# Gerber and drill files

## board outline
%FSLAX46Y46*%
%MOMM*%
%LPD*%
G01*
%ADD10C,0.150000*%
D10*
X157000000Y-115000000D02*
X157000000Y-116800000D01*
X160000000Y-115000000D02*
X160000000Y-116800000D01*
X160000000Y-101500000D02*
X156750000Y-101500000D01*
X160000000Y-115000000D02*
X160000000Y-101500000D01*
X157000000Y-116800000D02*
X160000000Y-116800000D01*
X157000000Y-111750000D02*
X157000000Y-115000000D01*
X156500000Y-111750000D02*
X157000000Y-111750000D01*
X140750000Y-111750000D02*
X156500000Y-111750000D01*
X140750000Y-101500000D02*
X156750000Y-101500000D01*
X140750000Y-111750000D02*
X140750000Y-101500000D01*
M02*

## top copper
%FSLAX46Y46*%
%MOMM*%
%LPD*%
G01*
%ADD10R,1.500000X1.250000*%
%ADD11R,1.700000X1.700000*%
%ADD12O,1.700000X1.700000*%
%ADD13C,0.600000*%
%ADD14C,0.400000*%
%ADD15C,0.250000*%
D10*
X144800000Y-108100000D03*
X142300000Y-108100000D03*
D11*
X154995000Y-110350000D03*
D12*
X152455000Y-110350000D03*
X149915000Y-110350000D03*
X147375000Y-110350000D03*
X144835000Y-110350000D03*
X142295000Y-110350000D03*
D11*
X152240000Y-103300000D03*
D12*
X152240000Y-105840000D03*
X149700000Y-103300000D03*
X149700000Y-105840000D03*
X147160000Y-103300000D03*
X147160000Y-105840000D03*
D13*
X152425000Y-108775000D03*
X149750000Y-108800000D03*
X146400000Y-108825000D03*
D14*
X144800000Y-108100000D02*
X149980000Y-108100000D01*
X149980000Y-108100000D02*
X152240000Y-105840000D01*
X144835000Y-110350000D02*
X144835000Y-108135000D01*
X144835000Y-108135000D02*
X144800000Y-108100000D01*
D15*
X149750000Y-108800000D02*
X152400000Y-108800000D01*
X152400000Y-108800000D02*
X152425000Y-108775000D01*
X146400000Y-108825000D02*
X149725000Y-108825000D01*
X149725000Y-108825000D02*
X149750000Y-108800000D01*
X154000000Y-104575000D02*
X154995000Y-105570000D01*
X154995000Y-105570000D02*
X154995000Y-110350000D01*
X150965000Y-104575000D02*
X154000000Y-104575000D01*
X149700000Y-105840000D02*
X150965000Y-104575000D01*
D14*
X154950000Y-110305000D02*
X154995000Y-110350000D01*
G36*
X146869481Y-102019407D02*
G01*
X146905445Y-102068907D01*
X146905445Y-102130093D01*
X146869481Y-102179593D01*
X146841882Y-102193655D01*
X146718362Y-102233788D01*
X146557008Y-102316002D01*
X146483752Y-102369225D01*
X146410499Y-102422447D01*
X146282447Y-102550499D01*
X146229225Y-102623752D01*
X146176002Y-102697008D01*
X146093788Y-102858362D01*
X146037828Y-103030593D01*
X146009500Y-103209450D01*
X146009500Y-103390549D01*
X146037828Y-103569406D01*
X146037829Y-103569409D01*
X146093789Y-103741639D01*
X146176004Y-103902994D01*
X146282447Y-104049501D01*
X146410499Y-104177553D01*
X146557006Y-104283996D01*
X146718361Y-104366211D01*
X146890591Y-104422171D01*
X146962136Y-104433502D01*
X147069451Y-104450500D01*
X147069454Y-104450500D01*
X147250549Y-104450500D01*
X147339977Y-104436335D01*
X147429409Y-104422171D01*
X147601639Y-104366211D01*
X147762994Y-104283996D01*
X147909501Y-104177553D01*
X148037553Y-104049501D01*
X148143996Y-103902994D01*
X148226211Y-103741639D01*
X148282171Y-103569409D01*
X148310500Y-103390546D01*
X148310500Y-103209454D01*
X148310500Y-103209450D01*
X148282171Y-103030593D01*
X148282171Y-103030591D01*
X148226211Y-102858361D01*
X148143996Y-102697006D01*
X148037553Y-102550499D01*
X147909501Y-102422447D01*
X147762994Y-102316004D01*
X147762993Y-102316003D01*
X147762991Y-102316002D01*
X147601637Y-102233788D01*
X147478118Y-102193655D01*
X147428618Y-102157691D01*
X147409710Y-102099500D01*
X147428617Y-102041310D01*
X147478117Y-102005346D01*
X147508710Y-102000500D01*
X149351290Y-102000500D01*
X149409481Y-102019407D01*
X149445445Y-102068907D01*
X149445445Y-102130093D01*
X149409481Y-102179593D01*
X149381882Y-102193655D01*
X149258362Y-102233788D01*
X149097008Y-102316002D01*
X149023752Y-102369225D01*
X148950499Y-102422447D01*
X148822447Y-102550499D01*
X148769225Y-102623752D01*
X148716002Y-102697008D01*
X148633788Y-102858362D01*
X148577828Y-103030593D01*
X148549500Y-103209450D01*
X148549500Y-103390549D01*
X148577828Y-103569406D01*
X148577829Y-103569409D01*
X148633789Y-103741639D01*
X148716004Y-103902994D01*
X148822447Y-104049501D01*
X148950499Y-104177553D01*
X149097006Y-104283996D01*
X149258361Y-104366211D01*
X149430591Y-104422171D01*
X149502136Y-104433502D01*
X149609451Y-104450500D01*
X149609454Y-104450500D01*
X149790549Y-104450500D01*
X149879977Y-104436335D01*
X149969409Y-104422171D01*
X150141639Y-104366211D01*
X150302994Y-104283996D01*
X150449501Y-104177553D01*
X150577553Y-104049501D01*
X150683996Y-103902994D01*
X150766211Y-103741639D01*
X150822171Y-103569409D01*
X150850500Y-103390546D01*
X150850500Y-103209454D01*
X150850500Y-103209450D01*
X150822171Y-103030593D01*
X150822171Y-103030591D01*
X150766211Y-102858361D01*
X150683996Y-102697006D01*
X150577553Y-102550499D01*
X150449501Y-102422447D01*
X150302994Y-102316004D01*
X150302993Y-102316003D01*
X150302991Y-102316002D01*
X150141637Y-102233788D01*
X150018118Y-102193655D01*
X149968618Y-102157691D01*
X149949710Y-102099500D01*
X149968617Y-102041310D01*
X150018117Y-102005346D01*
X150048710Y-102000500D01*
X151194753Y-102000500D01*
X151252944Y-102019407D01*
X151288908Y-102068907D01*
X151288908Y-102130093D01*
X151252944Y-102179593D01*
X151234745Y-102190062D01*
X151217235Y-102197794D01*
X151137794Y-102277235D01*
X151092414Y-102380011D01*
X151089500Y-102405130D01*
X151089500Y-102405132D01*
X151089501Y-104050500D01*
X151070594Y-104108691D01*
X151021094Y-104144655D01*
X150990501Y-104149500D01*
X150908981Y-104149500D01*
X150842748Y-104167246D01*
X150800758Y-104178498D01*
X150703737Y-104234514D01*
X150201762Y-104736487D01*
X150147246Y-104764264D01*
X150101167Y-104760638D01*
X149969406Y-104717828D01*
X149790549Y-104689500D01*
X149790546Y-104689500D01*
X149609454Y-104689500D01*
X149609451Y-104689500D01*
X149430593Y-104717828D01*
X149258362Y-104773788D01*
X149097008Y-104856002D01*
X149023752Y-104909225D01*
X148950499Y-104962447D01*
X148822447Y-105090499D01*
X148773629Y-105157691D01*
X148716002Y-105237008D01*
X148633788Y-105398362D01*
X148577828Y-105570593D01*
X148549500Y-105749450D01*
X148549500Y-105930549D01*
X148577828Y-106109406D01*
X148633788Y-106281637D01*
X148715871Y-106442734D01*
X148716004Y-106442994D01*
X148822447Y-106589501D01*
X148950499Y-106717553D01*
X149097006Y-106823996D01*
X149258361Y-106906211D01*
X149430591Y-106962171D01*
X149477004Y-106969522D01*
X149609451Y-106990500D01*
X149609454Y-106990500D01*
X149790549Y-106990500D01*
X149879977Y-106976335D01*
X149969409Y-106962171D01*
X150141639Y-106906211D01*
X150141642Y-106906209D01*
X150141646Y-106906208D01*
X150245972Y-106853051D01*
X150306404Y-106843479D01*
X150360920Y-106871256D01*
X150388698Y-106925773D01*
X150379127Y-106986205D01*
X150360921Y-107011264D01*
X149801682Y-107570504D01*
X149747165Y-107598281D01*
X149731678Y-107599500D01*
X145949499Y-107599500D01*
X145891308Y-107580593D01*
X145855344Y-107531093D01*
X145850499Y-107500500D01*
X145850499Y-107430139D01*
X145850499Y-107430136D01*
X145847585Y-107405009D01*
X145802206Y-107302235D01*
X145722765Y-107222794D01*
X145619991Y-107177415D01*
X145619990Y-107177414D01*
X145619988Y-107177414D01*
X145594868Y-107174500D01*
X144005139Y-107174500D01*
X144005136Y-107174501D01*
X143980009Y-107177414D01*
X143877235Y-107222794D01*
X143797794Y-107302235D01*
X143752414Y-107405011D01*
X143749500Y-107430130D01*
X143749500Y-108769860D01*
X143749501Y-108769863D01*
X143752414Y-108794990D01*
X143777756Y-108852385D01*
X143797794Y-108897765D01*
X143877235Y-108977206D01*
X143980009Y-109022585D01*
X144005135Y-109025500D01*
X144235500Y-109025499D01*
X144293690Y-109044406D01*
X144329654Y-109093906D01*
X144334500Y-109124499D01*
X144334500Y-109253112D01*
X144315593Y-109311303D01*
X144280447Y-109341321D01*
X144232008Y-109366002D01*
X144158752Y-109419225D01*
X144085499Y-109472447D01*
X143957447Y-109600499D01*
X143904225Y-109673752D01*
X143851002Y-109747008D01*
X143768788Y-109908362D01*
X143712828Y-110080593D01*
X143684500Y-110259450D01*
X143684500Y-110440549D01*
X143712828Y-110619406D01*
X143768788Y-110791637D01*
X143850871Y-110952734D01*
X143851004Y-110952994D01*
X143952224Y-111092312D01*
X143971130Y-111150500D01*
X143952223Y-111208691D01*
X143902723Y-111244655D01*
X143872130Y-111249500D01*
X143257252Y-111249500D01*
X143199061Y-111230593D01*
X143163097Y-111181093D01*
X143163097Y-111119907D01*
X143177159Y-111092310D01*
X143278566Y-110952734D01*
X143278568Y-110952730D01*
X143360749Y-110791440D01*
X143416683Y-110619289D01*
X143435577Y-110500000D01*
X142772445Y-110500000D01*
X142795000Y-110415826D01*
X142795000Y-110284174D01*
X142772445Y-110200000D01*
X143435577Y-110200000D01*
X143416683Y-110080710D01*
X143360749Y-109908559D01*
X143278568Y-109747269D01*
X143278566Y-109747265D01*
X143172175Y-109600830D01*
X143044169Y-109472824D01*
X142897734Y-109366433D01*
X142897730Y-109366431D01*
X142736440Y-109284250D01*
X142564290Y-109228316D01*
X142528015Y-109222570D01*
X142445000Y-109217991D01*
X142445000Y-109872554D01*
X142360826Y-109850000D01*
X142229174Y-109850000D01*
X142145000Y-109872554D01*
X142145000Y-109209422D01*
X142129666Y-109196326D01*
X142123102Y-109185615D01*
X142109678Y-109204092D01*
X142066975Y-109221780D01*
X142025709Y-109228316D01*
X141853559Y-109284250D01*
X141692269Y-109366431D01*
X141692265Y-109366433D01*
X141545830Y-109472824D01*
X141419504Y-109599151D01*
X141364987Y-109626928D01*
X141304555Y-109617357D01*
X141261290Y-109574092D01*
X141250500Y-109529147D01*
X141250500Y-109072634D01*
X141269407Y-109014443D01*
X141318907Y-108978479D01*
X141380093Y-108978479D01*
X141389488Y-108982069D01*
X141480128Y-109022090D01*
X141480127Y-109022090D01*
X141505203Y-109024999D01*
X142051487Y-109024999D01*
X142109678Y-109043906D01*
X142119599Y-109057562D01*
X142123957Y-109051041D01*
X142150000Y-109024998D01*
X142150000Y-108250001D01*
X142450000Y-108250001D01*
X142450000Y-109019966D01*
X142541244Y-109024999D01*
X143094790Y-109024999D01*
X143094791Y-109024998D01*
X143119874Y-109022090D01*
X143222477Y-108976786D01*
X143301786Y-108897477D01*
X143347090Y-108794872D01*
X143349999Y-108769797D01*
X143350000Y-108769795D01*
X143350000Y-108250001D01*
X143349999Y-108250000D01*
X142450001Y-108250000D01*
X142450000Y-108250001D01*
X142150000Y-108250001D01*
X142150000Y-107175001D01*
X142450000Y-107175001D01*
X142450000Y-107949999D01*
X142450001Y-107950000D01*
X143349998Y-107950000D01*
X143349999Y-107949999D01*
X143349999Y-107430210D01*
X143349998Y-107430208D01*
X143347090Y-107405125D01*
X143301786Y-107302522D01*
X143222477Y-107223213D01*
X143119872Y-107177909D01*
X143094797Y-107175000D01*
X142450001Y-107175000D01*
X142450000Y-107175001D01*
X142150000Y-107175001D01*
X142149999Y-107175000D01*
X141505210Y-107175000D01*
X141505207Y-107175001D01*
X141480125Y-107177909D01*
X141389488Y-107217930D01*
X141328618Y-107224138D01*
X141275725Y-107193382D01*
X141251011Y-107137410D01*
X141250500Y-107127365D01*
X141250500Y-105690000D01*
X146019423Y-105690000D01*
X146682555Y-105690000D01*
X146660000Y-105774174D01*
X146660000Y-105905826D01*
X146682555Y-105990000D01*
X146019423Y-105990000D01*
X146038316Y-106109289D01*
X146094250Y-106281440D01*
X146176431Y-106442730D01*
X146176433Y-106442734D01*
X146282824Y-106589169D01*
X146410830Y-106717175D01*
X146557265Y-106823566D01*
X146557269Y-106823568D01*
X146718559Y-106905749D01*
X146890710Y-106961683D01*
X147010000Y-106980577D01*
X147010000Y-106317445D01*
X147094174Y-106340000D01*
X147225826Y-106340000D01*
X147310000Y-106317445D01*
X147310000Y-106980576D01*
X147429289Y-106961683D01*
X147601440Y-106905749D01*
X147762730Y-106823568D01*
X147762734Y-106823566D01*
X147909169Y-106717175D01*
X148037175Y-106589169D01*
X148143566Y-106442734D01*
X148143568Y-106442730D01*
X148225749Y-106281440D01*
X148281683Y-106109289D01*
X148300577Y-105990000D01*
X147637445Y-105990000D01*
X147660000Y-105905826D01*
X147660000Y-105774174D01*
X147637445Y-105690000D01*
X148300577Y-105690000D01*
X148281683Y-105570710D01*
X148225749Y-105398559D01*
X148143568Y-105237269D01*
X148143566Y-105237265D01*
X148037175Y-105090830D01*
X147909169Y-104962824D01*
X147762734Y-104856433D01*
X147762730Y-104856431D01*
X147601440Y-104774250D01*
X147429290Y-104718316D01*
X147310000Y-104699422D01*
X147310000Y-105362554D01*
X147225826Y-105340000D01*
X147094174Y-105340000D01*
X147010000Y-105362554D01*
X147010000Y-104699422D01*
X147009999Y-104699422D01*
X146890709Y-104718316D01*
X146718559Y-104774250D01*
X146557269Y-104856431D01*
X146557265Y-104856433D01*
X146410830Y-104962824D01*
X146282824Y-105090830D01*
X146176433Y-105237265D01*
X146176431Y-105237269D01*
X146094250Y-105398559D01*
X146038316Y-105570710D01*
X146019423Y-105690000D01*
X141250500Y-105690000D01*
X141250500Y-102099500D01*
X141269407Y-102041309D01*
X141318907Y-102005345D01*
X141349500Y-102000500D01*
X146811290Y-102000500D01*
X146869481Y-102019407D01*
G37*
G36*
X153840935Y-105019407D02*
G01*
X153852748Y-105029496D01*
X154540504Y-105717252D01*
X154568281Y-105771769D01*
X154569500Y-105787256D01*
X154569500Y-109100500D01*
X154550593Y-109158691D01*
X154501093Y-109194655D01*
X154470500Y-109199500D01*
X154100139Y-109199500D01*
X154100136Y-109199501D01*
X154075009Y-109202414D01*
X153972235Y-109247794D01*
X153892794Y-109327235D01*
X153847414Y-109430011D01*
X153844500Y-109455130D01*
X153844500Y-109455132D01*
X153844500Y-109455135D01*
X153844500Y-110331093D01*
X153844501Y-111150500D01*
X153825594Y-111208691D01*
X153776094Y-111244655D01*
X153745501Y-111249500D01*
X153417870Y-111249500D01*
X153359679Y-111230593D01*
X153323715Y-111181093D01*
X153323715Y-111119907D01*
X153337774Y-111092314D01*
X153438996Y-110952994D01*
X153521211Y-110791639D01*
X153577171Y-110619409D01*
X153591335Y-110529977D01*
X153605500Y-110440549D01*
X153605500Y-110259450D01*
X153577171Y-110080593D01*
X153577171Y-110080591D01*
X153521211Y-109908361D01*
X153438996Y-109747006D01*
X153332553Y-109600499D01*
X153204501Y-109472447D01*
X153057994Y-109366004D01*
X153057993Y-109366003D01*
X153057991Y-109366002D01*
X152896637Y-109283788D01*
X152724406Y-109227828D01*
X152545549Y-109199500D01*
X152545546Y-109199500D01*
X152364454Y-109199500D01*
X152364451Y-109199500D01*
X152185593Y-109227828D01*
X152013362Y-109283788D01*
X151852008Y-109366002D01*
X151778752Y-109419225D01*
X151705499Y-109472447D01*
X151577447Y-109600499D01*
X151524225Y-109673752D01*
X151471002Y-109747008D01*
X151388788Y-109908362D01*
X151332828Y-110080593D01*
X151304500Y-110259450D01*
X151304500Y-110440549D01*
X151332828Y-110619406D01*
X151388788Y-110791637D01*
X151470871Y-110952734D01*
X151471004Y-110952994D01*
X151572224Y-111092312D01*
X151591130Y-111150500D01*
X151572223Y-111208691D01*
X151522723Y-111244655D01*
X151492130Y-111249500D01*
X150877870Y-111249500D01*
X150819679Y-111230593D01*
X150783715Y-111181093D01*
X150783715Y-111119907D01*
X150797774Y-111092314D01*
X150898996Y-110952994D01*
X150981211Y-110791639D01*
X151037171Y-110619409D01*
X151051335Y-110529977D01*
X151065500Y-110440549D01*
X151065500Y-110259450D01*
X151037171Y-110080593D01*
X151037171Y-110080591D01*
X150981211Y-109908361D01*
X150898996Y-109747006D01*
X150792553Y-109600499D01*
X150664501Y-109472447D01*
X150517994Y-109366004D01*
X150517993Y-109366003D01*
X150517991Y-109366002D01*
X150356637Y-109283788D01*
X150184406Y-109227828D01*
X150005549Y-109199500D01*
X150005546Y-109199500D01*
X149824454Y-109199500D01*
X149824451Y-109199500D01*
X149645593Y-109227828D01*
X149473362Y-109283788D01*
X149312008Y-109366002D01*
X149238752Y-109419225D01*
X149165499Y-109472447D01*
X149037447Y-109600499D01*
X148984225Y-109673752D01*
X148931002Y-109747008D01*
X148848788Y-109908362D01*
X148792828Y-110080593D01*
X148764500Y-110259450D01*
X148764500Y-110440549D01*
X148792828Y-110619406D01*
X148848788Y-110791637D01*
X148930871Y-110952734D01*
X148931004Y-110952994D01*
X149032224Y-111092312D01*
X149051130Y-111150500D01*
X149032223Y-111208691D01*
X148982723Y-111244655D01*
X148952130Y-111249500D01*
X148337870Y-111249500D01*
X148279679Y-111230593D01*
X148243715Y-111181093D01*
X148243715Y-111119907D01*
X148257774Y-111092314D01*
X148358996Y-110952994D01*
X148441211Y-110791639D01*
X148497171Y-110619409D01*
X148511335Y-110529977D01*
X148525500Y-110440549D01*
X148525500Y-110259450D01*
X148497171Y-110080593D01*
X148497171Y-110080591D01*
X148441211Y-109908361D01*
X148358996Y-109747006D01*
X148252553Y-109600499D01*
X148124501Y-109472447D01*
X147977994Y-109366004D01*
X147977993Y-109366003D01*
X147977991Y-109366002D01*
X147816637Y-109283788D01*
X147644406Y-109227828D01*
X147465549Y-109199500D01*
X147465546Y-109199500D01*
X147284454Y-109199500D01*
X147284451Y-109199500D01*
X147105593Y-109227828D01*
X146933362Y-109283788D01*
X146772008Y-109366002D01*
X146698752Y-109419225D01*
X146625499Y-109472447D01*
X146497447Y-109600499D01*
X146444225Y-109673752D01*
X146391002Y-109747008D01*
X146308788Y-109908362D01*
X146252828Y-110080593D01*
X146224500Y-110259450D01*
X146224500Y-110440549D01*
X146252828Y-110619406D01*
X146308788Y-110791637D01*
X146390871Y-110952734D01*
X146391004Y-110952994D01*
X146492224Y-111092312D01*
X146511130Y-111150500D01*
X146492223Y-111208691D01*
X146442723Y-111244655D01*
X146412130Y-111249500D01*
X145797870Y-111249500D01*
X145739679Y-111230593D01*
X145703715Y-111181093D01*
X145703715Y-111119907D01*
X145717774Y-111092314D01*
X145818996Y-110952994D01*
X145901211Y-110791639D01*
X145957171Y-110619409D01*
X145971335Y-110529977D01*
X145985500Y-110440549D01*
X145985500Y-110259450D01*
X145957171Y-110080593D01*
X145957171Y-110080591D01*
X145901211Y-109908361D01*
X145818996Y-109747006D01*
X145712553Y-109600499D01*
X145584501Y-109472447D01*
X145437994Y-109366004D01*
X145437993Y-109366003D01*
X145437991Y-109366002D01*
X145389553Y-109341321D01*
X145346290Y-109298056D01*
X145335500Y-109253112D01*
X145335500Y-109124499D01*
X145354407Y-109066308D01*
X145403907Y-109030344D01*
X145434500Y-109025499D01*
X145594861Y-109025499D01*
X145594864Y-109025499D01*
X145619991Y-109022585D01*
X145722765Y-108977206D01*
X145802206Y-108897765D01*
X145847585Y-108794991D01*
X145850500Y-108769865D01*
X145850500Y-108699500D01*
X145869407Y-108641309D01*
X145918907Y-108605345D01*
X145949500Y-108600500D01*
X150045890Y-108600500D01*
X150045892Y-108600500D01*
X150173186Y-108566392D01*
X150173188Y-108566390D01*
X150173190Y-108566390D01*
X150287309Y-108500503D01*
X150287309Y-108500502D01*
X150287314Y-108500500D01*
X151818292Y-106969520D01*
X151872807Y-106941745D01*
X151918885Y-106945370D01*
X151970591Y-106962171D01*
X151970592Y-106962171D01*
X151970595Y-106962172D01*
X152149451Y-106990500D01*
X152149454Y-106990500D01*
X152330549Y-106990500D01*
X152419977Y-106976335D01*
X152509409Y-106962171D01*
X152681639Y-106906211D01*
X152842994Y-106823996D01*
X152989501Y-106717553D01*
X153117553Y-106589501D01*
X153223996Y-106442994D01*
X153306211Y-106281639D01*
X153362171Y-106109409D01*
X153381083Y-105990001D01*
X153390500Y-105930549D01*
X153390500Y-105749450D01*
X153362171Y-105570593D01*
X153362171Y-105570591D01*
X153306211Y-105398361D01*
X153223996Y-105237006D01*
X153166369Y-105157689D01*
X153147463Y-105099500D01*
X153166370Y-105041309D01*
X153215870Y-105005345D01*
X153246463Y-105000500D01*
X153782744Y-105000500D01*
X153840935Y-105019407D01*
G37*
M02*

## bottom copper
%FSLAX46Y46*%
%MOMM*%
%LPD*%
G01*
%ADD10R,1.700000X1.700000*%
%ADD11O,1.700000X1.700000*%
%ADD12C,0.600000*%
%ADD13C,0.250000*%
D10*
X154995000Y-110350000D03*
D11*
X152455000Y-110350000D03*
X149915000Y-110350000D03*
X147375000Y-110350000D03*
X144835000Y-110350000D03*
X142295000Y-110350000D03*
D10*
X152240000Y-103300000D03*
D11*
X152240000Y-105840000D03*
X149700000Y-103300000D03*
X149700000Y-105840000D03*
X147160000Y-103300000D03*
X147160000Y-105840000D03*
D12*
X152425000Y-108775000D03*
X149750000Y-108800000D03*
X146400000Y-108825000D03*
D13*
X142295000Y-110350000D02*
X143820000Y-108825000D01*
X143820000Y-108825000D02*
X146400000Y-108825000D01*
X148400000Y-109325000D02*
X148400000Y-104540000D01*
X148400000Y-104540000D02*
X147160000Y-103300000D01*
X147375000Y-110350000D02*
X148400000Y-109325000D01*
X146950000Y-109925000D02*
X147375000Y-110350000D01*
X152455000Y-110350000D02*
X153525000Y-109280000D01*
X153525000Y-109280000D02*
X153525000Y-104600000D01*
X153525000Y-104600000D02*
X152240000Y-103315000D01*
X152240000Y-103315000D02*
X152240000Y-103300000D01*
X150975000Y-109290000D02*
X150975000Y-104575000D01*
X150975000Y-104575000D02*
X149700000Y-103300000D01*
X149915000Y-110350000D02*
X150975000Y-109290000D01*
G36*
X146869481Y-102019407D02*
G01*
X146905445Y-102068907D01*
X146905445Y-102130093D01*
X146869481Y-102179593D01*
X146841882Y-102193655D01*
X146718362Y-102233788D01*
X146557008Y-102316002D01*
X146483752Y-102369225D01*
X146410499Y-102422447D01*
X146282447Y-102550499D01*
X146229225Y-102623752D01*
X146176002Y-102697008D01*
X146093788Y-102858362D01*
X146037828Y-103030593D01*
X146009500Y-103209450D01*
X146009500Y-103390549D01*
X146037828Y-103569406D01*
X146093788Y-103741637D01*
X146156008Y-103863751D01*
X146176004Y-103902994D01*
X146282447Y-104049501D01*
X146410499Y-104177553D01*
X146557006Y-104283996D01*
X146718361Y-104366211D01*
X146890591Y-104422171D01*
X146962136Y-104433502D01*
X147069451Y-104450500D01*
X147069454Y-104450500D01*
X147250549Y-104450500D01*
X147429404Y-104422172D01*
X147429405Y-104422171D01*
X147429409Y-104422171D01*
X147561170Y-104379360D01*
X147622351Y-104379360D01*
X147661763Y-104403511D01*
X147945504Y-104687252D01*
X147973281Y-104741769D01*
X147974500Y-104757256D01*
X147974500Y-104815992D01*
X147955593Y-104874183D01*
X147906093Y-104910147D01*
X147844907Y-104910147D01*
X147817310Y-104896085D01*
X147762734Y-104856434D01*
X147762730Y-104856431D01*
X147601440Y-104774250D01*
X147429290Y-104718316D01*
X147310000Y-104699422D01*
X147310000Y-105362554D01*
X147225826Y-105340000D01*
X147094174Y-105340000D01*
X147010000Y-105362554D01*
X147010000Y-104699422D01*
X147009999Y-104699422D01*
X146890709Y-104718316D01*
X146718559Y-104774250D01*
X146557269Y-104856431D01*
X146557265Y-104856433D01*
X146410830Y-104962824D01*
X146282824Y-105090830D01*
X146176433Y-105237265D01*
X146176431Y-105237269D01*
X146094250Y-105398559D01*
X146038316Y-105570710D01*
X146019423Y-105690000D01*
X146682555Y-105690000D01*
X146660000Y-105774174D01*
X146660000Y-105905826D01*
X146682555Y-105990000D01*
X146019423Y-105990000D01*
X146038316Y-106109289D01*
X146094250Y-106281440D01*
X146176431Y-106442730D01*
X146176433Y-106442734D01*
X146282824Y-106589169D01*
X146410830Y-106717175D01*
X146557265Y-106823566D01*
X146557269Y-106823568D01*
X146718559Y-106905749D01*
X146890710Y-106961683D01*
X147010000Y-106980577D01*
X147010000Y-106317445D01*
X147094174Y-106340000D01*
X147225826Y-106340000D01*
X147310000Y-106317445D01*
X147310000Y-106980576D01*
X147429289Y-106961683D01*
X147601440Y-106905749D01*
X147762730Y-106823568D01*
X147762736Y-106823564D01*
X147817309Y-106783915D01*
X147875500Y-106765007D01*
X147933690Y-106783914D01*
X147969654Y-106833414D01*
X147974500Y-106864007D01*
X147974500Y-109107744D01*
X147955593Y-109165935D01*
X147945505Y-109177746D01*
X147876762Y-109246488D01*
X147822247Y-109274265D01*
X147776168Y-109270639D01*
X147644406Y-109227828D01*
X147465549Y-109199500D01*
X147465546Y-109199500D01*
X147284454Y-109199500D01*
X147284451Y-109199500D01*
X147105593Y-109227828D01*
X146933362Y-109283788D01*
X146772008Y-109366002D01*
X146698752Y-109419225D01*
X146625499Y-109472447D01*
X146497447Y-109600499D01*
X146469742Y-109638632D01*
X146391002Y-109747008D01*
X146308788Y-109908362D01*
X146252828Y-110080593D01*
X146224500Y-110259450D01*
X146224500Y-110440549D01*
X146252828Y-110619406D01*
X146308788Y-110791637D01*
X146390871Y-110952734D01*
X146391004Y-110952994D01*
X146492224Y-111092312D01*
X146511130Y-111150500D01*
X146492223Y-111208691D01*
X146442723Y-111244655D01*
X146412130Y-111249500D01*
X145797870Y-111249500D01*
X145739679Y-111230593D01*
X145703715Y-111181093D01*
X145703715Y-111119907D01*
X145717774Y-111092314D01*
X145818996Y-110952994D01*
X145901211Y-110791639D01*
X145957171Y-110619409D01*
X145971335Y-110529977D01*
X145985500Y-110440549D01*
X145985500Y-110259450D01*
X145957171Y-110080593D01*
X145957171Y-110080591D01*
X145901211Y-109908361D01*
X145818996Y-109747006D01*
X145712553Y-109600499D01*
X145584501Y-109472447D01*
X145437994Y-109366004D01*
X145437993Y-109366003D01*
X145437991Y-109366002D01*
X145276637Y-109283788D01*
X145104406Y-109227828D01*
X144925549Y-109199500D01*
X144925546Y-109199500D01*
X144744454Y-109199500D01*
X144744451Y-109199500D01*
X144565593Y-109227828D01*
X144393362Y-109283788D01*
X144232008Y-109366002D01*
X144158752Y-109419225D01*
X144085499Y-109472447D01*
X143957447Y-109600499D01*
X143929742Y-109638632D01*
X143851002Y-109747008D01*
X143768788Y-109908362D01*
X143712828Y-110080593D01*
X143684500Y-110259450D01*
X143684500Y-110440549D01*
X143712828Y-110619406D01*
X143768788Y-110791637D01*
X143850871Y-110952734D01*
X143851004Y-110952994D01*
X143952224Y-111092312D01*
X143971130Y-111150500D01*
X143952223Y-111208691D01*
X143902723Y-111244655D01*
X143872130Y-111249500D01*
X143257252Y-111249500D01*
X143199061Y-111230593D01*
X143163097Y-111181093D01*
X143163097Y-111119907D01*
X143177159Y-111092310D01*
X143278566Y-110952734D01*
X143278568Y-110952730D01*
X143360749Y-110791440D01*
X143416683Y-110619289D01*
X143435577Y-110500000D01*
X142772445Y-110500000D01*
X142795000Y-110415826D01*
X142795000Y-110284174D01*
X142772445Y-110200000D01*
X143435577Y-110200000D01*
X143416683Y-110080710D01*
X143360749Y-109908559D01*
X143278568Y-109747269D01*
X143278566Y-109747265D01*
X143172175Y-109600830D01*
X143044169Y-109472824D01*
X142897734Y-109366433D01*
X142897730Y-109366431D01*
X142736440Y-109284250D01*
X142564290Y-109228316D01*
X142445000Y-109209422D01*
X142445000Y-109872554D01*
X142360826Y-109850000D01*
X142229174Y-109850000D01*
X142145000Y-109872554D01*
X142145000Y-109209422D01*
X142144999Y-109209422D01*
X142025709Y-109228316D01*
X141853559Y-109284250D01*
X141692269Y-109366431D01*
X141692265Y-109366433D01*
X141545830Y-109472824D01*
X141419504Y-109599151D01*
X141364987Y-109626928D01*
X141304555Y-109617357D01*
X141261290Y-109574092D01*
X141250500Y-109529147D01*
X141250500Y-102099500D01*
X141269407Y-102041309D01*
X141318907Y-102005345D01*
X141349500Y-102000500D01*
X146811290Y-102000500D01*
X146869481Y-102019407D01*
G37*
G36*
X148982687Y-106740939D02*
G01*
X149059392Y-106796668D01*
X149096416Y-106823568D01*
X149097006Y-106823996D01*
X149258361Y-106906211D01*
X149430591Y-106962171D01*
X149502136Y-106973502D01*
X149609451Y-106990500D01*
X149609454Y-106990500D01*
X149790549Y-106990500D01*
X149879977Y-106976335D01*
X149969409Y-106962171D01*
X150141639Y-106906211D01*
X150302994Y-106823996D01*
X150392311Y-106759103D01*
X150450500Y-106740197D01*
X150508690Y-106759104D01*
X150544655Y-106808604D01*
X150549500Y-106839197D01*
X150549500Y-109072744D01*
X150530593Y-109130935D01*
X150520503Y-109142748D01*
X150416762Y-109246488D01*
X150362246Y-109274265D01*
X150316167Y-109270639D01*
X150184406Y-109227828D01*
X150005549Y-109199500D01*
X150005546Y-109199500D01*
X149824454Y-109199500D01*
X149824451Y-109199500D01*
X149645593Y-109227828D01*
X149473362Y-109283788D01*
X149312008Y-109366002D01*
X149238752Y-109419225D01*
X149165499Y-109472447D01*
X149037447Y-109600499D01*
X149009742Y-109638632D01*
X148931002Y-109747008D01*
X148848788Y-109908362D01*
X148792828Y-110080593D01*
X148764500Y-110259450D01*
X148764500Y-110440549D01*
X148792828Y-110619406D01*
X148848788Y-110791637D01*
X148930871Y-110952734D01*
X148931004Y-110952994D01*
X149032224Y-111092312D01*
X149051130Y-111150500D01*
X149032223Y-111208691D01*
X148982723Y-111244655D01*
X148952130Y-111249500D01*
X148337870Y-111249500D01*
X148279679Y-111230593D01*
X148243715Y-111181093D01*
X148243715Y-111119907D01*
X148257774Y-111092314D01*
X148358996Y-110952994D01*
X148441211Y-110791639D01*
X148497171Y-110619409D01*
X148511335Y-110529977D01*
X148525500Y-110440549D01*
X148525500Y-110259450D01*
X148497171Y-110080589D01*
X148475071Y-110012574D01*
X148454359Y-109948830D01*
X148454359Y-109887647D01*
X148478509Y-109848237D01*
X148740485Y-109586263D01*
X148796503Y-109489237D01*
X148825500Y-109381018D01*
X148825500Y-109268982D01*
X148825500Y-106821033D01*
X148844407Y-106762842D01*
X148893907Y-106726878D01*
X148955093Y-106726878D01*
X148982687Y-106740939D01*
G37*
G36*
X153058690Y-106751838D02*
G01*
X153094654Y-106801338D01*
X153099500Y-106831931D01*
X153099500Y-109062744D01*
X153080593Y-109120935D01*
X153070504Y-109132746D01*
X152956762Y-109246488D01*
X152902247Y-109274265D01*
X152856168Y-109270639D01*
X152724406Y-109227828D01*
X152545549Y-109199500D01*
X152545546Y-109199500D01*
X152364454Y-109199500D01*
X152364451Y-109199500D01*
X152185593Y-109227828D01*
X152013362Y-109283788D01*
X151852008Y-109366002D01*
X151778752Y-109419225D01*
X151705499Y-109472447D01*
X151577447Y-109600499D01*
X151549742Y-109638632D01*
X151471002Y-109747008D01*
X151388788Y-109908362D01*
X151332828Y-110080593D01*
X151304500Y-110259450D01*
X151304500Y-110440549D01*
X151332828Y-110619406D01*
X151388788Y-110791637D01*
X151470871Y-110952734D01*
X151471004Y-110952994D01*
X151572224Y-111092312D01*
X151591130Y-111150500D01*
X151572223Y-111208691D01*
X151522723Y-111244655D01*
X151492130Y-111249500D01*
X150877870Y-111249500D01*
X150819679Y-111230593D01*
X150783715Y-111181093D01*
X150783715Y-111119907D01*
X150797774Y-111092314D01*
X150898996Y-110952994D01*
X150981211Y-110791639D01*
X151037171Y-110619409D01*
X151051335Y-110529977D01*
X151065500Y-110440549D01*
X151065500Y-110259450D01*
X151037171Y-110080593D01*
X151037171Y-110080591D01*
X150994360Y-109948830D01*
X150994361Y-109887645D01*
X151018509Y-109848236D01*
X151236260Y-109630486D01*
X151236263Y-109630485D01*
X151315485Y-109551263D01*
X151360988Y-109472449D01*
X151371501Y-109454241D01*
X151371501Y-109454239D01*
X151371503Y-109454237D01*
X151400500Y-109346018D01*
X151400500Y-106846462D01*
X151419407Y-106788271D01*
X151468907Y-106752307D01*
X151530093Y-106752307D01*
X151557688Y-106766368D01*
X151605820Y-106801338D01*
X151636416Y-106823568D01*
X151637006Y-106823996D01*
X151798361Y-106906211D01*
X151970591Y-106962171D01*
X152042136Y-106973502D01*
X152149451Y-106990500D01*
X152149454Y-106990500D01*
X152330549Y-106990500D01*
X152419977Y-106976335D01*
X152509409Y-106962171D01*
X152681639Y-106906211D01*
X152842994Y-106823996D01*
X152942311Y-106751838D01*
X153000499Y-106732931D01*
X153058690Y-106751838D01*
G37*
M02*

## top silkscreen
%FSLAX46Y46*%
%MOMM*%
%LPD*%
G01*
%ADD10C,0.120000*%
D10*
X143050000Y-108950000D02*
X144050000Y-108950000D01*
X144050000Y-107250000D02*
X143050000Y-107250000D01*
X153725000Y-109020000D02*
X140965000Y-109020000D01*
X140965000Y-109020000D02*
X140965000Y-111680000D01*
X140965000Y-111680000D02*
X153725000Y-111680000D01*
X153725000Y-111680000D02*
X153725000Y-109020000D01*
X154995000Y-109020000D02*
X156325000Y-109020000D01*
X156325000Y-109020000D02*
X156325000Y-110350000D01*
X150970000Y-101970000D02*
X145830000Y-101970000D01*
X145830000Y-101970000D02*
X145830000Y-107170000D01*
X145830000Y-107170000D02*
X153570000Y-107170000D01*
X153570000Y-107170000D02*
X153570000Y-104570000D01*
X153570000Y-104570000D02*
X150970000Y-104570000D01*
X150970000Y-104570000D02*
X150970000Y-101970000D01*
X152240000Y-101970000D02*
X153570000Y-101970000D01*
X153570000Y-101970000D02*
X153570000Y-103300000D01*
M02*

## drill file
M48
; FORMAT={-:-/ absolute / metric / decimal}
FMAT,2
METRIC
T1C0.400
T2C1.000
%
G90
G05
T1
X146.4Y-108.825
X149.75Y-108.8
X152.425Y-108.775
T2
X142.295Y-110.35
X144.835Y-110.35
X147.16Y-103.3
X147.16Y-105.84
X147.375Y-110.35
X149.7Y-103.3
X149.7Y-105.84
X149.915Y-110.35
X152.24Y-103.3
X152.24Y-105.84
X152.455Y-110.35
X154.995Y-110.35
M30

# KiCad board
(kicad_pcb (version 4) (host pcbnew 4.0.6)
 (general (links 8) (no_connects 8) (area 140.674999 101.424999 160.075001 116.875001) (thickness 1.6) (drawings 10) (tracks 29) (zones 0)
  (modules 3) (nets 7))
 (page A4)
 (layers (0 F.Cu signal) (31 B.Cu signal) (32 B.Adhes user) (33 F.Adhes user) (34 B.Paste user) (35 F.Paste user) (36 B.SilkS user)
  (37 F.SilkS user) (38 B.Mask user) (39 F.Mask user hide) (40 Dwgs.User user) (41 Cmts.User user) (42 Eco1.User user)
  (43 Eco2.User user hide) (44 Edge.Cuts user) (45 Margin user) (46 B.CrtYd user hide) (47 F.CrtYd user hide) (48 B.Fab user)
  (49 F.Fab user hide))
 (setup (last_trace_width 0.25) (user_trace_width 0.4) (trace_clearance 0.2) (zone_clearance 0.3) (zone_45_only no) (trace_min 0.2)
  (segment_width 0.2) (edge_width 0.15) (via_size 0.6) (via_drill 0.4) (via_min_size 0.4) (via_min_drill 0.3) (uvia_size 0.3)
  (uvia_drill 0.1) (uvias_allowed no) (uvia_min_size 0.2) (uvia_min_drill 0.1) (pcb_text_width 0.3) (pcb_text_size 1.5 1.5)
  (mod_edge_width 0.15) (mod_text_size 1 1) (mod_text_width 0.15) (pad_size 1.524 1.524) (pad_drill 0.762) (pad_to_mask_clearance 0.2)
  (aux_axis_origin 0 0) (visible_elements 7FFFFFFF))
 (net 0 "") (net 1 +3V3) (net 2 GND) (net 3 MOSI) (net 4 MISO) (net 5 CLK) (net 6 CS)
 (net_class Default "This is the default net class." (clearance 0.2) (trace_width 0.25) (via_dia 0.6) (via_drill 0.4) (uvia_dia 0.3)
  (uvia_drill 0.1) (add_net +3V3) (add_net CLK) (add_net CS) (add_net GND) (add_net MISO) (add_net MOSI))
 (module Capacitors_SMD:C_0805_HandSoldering (layer F.Cu) (at 143.55 108.1 180)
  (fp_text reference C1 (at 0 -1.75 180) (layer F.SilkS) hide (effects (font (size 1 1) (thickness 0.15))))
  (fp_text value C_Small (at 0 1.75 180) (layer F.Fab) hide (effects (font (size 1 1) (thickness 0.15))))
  (fp_line (start 0.5 -0.85) (end -0.5 -0.85) (layer F.SilkS) (width 0.12))
  (fp_line (start -0.5 0.85) (end 0.5 0.85) (layer F.SilkS) (width 0.12))
  (pad 1 smd rect (at -1.25 0 180) (size 1.5 1.25) (layers F.Cu F.Paste F.Mask) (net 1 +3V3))
  (pad 2 smd rect (at 1.25 0 180) (size 1.5 1.25) (layers F.Cu F.Paste F.Mask) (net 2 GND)))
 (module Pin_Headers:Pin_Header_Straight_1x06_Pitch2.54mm (layer F.Cu) (at 154.995 110.35 270)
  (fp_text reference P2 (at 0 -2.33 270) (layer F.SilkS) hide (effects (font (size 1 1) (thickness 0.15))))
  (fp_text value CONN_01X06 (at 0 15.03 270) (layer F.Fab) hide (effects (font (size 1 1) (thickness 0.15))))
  (fp_line (start -1.33 1.27) (end -1.33 14.03) (layer F.SilkS) (width 0.12))
  (fp_line (start -1.33 14.03) (end 1.33 14.03) (layer F.SilkS) (width 0.12))
  (fp_line (start 1.33 14.03) (end 1.33 1.27) (layer F.SilkS) (width 0.12))
  (fp_line (start 1.33 1.27) (end -1.33 1.27) (layer F.SilkS) (width 0.12))
  (fp_line (start -1.33 0) (end -1.33 -1.33) (layer F.SilkS) (width 0.12))
  (fp_line (start -1.33 -1.33) (end 0 -1.33) (layer F.SilkS) (width 0.12))
  (pad 1 thru_hole rect (at 0 0 270) (size 1.7 1.7) (drill 1) (layers *.Cu *.Mask) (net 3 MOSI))
  (pad 2 thru_hole oval (at 0 2.54 270) (size 1.7 1.7) (drill 1) (layers *.Cu *.Mask) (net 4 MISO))
  (pad 3 thru_hole oval (at 0 5.08 270) (size 1.7 1.7) (drill 1) (layers *.Cu *.Mask) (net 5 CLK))
  (pad 4 thru_hole oval (at 0 7.62 270) (size 1.7 1.7) (drill 1) (layers *.Cu *.Mask) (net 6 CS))
  (pad 5 thru_hole oval (at 0 10.16 270) (size 1.7 1.7) (drill 1) (layers *.Cu *.Mask) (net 1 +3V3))
  (pad 6 thru_hole oval (at 0 12.7 270) (size 1.7 1.7) (drill 1) (layers *.Cu *.Mask) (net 2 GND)))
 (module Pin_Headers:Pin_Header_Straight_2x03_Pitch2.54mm (layer F.Cu) (at 152.24 103.3 270)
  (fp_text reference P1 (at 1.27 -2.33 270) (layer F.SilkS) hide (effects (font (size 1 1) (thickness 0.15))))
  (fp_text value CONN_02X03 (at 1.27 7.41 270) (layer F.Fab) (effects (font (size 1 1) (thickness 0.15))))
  (fp_line (start -1.33 1.27) (end -1.33 6.41) (layer F.SilkS) (width 0.12))
  (fp_line (start -1.33 6.41) (end 3.87 6.41) (layer F.SilkS) (width 0.12))
  (fp_line (start 3.87 6.41) (end 3.87 -1.33) (layer F.SilkS) (width 0.12))
  (fp_line (start 3.87 -1.33) (end 1.27 -1.33) (layer F.SilkS) (width 0.12))
  (fp_line (start 1.27 -1.33) (end 1.27 1.27) (layer F.SilkS) (width 0.12))
  (fp_line (start 1.27 1.27) (end -1.33 1.27) (layer F.SilkS) (width 0.12))
  (fp_line (start -1.33 0) (end -1.33 -1.33) (layer F.SilkS) (width 0.12))
  (fp_line (start -1.33 -1.33) (end 0 -1.33) (layer F.SilkS) (width 0.12))
  (pad 1 thru_hole rect (at 0 0 270) (size 1.7 1.7) (drill 1) (layers *.Cu *.Mask) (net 4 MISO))
  (pad 2 thru_hole oval (at 2.54 0 270) (size 1.7 1.7) (drill 1) (layers *.Cu *.Mask) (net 1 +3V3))
  (pad 3 thru_hole oval (at 0 2.54 270) (size 1.7 1.7) (drill 1) (layers *.Cu *.Mask) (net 5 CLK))
  (pad 4 thru_hole oval (at 2.54 2.54 270) (size 1.7 1.7) (drill 1) (layers *.Cu *.Mask) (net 3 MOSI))
  (pad 5 thru_hole oval (at 0 5.08 270) (size 1.7 1.7) (drill 1) (layers *.Cu *.Mask) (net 6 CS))
  (pad 6 thru_hole oval (at 2.54 5.08 270) (size 1.7 1.7) (drill 1) (layers *.Cu *.Mask) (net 2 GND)))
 (gr_line (start 157 115) (end 157 116.8) (layer Edge.Cuts) (width 0.15))
 (gr_line (start 160 115) (end 160 116.8) (layer Edge.Cuts) (width 0.15))
 (gr_line (start 160 101.5) (end 156.75 101.5) (layer Edge.Cuts) (width 0.15))
 (gr_line (start 160 115) (end 160 101.5) (layer Edge.Cuts) (width 0.15))
 (gr_line (start 157 116.8) (end 160 116.8) (layer Edge.Cuts) (width 0.15))
 (gr_line (start 157 111.75) (end 157 115) (layer Edge.Cuts) (width 0.15))
 (gr_line (start 156.5 111.75) (end 157 111.75) (layer Edge.Cuts) (width 0.15))
 (gr_line (start 140.75 111.75) (end 156.5 111.75) (layer Edge.Cuts) (width 0.15))
 (gr_line (start 140.75 101.5) (end 156.75 101.5) (layer Edge.Cuts) (width 0.15))
 (gr_line (start 140.75 111.75) (end 140.75 101.5) (layer Edge.Cuts) (width 0.15))
 (segment (start 144.8 108.1) (end 149.98 108.1) (width 0.4) (layer F.Cu) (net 1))
 (segment (start 149.98 108.1) (end 152.24 105.84) (width 0.4) (layer F.Cu) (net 1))
 (segment (start 144.835 110.35) (end 144.835 108.135) (width 0.4) (layer F.Cu) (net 1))
 (segment (start 144.835 108.135) (end 144.8 108.1) (width 0.4) (layer F.Cu) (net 1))
 (segment (start 149.75 108.8) (end 152.4 108.8) (width 0.25) (layer F.Cu) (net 2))
 (segment (start 152.4 108.8) (end 152.425 108.775) (width 0.25) (layer F.Cu) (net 2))
 (via (at 152.425 108.775) (size 0.6) (drill 0.4) (layers F.Cu B.Cu) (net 2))
 (segment (start 146.4 108.825) (end 149.725 108.825) (width 0.25) (layer F.Cu) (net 2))
 (segment (start 149.725 108.825) (end 149.75 108.8) (width 0.25) (layer F.Cu) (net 2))
 (via (at 149.75 108.8) (size 0.6) (drill 0.4) (layers F.Cu B.Cu) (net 2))
 (segment (start 142.295 110.35) (end 143.82 108.825) (width 0.25) (layer B.Cu) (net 2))
 (segment (start 143.82 108.825) (end 146.4 108.825) (width 0.25) (layer B.Cu) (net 2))
 (via (at 146.4 108.825) (size 0.6) (drill 0.4) (layers F.Cu B.Cu) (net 2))
 (segment (start 148.4 109.325) (end 148.4 104.54) (width 0.25) (layer B.Cu) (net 6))
 (segment (start 148.4 104.54) (end 147.16 103.3) (width 0.25) (layer B.Cu) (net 6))
 (segment (start 147.375 110.35) (end 148.4 109.325) (width 0.25) (layer B.Cu) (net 6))
 (segment (start 146.95 109.925) (end 147.375 110.35) (width 0.25) (layer B.Cu) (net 6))
 (segment (start 152.455 110.35) (end 153.525 109.28) (width 0.25) (layer B.Cu) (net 4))
 (segment (start 153.525 109.28) (end 153.525 104.6) (width 0.25) (layer B.Cu) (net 4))
 (segment (start 153.525 104.6) (end 152.24 103.315) (width 0.25) (layer B.Cu) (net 4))
 (segment (start 152.24 103.315) (end 152.24 103.3) (width 0.25) (layer B.Cu) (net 4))
 (segment (start 150.975 109.29) (end 150.975 104.575) (width 0.25) (layer B.Cu) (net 5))
 (segment (start 150.975 104.575) (end 149.7 103.3) (width 0.25) (layer B.Cu) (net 5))
 (segment (start 149.915 110.35) (end 150.975 109.29) (width 0.25) (layer B.Cu) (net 5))
 (segment (start 154 104.575) (end 154.995 105.57) (width 0.25) (layer F.Cu) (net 3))
 (segment (start 154.995 105.57) (end 154.995 110.35) (width 0.25) (layer F.Cu) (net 3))
 (segment (start 150.965 104.575) (end 154 104.575) (width 0.25) (layer F.Cu) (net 3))
 (segment (start 149.7 105.84) (end 150.965 104.575) (width 0.25) (layer F.Cu) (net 3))
 (segment (start 154.95 110.305) (end 154.995 110.35) (width 0.4) (layer F.Cu) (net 3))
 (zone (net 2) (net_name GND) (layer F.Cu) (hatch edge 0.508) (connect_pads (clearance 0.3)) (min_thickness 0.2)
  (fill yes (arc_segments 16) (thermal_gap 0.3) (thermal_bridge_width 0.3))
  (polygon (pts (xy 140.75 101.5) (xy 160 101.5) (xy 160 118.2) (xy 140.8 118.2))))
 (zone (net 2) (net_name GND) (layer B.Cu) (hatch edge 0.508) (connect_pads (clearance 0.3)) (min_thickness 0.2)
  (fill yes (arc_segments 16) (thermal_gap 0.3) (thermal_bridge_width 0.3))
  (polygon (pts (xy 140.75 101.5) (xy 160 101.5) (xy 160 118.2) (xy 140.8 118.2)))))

